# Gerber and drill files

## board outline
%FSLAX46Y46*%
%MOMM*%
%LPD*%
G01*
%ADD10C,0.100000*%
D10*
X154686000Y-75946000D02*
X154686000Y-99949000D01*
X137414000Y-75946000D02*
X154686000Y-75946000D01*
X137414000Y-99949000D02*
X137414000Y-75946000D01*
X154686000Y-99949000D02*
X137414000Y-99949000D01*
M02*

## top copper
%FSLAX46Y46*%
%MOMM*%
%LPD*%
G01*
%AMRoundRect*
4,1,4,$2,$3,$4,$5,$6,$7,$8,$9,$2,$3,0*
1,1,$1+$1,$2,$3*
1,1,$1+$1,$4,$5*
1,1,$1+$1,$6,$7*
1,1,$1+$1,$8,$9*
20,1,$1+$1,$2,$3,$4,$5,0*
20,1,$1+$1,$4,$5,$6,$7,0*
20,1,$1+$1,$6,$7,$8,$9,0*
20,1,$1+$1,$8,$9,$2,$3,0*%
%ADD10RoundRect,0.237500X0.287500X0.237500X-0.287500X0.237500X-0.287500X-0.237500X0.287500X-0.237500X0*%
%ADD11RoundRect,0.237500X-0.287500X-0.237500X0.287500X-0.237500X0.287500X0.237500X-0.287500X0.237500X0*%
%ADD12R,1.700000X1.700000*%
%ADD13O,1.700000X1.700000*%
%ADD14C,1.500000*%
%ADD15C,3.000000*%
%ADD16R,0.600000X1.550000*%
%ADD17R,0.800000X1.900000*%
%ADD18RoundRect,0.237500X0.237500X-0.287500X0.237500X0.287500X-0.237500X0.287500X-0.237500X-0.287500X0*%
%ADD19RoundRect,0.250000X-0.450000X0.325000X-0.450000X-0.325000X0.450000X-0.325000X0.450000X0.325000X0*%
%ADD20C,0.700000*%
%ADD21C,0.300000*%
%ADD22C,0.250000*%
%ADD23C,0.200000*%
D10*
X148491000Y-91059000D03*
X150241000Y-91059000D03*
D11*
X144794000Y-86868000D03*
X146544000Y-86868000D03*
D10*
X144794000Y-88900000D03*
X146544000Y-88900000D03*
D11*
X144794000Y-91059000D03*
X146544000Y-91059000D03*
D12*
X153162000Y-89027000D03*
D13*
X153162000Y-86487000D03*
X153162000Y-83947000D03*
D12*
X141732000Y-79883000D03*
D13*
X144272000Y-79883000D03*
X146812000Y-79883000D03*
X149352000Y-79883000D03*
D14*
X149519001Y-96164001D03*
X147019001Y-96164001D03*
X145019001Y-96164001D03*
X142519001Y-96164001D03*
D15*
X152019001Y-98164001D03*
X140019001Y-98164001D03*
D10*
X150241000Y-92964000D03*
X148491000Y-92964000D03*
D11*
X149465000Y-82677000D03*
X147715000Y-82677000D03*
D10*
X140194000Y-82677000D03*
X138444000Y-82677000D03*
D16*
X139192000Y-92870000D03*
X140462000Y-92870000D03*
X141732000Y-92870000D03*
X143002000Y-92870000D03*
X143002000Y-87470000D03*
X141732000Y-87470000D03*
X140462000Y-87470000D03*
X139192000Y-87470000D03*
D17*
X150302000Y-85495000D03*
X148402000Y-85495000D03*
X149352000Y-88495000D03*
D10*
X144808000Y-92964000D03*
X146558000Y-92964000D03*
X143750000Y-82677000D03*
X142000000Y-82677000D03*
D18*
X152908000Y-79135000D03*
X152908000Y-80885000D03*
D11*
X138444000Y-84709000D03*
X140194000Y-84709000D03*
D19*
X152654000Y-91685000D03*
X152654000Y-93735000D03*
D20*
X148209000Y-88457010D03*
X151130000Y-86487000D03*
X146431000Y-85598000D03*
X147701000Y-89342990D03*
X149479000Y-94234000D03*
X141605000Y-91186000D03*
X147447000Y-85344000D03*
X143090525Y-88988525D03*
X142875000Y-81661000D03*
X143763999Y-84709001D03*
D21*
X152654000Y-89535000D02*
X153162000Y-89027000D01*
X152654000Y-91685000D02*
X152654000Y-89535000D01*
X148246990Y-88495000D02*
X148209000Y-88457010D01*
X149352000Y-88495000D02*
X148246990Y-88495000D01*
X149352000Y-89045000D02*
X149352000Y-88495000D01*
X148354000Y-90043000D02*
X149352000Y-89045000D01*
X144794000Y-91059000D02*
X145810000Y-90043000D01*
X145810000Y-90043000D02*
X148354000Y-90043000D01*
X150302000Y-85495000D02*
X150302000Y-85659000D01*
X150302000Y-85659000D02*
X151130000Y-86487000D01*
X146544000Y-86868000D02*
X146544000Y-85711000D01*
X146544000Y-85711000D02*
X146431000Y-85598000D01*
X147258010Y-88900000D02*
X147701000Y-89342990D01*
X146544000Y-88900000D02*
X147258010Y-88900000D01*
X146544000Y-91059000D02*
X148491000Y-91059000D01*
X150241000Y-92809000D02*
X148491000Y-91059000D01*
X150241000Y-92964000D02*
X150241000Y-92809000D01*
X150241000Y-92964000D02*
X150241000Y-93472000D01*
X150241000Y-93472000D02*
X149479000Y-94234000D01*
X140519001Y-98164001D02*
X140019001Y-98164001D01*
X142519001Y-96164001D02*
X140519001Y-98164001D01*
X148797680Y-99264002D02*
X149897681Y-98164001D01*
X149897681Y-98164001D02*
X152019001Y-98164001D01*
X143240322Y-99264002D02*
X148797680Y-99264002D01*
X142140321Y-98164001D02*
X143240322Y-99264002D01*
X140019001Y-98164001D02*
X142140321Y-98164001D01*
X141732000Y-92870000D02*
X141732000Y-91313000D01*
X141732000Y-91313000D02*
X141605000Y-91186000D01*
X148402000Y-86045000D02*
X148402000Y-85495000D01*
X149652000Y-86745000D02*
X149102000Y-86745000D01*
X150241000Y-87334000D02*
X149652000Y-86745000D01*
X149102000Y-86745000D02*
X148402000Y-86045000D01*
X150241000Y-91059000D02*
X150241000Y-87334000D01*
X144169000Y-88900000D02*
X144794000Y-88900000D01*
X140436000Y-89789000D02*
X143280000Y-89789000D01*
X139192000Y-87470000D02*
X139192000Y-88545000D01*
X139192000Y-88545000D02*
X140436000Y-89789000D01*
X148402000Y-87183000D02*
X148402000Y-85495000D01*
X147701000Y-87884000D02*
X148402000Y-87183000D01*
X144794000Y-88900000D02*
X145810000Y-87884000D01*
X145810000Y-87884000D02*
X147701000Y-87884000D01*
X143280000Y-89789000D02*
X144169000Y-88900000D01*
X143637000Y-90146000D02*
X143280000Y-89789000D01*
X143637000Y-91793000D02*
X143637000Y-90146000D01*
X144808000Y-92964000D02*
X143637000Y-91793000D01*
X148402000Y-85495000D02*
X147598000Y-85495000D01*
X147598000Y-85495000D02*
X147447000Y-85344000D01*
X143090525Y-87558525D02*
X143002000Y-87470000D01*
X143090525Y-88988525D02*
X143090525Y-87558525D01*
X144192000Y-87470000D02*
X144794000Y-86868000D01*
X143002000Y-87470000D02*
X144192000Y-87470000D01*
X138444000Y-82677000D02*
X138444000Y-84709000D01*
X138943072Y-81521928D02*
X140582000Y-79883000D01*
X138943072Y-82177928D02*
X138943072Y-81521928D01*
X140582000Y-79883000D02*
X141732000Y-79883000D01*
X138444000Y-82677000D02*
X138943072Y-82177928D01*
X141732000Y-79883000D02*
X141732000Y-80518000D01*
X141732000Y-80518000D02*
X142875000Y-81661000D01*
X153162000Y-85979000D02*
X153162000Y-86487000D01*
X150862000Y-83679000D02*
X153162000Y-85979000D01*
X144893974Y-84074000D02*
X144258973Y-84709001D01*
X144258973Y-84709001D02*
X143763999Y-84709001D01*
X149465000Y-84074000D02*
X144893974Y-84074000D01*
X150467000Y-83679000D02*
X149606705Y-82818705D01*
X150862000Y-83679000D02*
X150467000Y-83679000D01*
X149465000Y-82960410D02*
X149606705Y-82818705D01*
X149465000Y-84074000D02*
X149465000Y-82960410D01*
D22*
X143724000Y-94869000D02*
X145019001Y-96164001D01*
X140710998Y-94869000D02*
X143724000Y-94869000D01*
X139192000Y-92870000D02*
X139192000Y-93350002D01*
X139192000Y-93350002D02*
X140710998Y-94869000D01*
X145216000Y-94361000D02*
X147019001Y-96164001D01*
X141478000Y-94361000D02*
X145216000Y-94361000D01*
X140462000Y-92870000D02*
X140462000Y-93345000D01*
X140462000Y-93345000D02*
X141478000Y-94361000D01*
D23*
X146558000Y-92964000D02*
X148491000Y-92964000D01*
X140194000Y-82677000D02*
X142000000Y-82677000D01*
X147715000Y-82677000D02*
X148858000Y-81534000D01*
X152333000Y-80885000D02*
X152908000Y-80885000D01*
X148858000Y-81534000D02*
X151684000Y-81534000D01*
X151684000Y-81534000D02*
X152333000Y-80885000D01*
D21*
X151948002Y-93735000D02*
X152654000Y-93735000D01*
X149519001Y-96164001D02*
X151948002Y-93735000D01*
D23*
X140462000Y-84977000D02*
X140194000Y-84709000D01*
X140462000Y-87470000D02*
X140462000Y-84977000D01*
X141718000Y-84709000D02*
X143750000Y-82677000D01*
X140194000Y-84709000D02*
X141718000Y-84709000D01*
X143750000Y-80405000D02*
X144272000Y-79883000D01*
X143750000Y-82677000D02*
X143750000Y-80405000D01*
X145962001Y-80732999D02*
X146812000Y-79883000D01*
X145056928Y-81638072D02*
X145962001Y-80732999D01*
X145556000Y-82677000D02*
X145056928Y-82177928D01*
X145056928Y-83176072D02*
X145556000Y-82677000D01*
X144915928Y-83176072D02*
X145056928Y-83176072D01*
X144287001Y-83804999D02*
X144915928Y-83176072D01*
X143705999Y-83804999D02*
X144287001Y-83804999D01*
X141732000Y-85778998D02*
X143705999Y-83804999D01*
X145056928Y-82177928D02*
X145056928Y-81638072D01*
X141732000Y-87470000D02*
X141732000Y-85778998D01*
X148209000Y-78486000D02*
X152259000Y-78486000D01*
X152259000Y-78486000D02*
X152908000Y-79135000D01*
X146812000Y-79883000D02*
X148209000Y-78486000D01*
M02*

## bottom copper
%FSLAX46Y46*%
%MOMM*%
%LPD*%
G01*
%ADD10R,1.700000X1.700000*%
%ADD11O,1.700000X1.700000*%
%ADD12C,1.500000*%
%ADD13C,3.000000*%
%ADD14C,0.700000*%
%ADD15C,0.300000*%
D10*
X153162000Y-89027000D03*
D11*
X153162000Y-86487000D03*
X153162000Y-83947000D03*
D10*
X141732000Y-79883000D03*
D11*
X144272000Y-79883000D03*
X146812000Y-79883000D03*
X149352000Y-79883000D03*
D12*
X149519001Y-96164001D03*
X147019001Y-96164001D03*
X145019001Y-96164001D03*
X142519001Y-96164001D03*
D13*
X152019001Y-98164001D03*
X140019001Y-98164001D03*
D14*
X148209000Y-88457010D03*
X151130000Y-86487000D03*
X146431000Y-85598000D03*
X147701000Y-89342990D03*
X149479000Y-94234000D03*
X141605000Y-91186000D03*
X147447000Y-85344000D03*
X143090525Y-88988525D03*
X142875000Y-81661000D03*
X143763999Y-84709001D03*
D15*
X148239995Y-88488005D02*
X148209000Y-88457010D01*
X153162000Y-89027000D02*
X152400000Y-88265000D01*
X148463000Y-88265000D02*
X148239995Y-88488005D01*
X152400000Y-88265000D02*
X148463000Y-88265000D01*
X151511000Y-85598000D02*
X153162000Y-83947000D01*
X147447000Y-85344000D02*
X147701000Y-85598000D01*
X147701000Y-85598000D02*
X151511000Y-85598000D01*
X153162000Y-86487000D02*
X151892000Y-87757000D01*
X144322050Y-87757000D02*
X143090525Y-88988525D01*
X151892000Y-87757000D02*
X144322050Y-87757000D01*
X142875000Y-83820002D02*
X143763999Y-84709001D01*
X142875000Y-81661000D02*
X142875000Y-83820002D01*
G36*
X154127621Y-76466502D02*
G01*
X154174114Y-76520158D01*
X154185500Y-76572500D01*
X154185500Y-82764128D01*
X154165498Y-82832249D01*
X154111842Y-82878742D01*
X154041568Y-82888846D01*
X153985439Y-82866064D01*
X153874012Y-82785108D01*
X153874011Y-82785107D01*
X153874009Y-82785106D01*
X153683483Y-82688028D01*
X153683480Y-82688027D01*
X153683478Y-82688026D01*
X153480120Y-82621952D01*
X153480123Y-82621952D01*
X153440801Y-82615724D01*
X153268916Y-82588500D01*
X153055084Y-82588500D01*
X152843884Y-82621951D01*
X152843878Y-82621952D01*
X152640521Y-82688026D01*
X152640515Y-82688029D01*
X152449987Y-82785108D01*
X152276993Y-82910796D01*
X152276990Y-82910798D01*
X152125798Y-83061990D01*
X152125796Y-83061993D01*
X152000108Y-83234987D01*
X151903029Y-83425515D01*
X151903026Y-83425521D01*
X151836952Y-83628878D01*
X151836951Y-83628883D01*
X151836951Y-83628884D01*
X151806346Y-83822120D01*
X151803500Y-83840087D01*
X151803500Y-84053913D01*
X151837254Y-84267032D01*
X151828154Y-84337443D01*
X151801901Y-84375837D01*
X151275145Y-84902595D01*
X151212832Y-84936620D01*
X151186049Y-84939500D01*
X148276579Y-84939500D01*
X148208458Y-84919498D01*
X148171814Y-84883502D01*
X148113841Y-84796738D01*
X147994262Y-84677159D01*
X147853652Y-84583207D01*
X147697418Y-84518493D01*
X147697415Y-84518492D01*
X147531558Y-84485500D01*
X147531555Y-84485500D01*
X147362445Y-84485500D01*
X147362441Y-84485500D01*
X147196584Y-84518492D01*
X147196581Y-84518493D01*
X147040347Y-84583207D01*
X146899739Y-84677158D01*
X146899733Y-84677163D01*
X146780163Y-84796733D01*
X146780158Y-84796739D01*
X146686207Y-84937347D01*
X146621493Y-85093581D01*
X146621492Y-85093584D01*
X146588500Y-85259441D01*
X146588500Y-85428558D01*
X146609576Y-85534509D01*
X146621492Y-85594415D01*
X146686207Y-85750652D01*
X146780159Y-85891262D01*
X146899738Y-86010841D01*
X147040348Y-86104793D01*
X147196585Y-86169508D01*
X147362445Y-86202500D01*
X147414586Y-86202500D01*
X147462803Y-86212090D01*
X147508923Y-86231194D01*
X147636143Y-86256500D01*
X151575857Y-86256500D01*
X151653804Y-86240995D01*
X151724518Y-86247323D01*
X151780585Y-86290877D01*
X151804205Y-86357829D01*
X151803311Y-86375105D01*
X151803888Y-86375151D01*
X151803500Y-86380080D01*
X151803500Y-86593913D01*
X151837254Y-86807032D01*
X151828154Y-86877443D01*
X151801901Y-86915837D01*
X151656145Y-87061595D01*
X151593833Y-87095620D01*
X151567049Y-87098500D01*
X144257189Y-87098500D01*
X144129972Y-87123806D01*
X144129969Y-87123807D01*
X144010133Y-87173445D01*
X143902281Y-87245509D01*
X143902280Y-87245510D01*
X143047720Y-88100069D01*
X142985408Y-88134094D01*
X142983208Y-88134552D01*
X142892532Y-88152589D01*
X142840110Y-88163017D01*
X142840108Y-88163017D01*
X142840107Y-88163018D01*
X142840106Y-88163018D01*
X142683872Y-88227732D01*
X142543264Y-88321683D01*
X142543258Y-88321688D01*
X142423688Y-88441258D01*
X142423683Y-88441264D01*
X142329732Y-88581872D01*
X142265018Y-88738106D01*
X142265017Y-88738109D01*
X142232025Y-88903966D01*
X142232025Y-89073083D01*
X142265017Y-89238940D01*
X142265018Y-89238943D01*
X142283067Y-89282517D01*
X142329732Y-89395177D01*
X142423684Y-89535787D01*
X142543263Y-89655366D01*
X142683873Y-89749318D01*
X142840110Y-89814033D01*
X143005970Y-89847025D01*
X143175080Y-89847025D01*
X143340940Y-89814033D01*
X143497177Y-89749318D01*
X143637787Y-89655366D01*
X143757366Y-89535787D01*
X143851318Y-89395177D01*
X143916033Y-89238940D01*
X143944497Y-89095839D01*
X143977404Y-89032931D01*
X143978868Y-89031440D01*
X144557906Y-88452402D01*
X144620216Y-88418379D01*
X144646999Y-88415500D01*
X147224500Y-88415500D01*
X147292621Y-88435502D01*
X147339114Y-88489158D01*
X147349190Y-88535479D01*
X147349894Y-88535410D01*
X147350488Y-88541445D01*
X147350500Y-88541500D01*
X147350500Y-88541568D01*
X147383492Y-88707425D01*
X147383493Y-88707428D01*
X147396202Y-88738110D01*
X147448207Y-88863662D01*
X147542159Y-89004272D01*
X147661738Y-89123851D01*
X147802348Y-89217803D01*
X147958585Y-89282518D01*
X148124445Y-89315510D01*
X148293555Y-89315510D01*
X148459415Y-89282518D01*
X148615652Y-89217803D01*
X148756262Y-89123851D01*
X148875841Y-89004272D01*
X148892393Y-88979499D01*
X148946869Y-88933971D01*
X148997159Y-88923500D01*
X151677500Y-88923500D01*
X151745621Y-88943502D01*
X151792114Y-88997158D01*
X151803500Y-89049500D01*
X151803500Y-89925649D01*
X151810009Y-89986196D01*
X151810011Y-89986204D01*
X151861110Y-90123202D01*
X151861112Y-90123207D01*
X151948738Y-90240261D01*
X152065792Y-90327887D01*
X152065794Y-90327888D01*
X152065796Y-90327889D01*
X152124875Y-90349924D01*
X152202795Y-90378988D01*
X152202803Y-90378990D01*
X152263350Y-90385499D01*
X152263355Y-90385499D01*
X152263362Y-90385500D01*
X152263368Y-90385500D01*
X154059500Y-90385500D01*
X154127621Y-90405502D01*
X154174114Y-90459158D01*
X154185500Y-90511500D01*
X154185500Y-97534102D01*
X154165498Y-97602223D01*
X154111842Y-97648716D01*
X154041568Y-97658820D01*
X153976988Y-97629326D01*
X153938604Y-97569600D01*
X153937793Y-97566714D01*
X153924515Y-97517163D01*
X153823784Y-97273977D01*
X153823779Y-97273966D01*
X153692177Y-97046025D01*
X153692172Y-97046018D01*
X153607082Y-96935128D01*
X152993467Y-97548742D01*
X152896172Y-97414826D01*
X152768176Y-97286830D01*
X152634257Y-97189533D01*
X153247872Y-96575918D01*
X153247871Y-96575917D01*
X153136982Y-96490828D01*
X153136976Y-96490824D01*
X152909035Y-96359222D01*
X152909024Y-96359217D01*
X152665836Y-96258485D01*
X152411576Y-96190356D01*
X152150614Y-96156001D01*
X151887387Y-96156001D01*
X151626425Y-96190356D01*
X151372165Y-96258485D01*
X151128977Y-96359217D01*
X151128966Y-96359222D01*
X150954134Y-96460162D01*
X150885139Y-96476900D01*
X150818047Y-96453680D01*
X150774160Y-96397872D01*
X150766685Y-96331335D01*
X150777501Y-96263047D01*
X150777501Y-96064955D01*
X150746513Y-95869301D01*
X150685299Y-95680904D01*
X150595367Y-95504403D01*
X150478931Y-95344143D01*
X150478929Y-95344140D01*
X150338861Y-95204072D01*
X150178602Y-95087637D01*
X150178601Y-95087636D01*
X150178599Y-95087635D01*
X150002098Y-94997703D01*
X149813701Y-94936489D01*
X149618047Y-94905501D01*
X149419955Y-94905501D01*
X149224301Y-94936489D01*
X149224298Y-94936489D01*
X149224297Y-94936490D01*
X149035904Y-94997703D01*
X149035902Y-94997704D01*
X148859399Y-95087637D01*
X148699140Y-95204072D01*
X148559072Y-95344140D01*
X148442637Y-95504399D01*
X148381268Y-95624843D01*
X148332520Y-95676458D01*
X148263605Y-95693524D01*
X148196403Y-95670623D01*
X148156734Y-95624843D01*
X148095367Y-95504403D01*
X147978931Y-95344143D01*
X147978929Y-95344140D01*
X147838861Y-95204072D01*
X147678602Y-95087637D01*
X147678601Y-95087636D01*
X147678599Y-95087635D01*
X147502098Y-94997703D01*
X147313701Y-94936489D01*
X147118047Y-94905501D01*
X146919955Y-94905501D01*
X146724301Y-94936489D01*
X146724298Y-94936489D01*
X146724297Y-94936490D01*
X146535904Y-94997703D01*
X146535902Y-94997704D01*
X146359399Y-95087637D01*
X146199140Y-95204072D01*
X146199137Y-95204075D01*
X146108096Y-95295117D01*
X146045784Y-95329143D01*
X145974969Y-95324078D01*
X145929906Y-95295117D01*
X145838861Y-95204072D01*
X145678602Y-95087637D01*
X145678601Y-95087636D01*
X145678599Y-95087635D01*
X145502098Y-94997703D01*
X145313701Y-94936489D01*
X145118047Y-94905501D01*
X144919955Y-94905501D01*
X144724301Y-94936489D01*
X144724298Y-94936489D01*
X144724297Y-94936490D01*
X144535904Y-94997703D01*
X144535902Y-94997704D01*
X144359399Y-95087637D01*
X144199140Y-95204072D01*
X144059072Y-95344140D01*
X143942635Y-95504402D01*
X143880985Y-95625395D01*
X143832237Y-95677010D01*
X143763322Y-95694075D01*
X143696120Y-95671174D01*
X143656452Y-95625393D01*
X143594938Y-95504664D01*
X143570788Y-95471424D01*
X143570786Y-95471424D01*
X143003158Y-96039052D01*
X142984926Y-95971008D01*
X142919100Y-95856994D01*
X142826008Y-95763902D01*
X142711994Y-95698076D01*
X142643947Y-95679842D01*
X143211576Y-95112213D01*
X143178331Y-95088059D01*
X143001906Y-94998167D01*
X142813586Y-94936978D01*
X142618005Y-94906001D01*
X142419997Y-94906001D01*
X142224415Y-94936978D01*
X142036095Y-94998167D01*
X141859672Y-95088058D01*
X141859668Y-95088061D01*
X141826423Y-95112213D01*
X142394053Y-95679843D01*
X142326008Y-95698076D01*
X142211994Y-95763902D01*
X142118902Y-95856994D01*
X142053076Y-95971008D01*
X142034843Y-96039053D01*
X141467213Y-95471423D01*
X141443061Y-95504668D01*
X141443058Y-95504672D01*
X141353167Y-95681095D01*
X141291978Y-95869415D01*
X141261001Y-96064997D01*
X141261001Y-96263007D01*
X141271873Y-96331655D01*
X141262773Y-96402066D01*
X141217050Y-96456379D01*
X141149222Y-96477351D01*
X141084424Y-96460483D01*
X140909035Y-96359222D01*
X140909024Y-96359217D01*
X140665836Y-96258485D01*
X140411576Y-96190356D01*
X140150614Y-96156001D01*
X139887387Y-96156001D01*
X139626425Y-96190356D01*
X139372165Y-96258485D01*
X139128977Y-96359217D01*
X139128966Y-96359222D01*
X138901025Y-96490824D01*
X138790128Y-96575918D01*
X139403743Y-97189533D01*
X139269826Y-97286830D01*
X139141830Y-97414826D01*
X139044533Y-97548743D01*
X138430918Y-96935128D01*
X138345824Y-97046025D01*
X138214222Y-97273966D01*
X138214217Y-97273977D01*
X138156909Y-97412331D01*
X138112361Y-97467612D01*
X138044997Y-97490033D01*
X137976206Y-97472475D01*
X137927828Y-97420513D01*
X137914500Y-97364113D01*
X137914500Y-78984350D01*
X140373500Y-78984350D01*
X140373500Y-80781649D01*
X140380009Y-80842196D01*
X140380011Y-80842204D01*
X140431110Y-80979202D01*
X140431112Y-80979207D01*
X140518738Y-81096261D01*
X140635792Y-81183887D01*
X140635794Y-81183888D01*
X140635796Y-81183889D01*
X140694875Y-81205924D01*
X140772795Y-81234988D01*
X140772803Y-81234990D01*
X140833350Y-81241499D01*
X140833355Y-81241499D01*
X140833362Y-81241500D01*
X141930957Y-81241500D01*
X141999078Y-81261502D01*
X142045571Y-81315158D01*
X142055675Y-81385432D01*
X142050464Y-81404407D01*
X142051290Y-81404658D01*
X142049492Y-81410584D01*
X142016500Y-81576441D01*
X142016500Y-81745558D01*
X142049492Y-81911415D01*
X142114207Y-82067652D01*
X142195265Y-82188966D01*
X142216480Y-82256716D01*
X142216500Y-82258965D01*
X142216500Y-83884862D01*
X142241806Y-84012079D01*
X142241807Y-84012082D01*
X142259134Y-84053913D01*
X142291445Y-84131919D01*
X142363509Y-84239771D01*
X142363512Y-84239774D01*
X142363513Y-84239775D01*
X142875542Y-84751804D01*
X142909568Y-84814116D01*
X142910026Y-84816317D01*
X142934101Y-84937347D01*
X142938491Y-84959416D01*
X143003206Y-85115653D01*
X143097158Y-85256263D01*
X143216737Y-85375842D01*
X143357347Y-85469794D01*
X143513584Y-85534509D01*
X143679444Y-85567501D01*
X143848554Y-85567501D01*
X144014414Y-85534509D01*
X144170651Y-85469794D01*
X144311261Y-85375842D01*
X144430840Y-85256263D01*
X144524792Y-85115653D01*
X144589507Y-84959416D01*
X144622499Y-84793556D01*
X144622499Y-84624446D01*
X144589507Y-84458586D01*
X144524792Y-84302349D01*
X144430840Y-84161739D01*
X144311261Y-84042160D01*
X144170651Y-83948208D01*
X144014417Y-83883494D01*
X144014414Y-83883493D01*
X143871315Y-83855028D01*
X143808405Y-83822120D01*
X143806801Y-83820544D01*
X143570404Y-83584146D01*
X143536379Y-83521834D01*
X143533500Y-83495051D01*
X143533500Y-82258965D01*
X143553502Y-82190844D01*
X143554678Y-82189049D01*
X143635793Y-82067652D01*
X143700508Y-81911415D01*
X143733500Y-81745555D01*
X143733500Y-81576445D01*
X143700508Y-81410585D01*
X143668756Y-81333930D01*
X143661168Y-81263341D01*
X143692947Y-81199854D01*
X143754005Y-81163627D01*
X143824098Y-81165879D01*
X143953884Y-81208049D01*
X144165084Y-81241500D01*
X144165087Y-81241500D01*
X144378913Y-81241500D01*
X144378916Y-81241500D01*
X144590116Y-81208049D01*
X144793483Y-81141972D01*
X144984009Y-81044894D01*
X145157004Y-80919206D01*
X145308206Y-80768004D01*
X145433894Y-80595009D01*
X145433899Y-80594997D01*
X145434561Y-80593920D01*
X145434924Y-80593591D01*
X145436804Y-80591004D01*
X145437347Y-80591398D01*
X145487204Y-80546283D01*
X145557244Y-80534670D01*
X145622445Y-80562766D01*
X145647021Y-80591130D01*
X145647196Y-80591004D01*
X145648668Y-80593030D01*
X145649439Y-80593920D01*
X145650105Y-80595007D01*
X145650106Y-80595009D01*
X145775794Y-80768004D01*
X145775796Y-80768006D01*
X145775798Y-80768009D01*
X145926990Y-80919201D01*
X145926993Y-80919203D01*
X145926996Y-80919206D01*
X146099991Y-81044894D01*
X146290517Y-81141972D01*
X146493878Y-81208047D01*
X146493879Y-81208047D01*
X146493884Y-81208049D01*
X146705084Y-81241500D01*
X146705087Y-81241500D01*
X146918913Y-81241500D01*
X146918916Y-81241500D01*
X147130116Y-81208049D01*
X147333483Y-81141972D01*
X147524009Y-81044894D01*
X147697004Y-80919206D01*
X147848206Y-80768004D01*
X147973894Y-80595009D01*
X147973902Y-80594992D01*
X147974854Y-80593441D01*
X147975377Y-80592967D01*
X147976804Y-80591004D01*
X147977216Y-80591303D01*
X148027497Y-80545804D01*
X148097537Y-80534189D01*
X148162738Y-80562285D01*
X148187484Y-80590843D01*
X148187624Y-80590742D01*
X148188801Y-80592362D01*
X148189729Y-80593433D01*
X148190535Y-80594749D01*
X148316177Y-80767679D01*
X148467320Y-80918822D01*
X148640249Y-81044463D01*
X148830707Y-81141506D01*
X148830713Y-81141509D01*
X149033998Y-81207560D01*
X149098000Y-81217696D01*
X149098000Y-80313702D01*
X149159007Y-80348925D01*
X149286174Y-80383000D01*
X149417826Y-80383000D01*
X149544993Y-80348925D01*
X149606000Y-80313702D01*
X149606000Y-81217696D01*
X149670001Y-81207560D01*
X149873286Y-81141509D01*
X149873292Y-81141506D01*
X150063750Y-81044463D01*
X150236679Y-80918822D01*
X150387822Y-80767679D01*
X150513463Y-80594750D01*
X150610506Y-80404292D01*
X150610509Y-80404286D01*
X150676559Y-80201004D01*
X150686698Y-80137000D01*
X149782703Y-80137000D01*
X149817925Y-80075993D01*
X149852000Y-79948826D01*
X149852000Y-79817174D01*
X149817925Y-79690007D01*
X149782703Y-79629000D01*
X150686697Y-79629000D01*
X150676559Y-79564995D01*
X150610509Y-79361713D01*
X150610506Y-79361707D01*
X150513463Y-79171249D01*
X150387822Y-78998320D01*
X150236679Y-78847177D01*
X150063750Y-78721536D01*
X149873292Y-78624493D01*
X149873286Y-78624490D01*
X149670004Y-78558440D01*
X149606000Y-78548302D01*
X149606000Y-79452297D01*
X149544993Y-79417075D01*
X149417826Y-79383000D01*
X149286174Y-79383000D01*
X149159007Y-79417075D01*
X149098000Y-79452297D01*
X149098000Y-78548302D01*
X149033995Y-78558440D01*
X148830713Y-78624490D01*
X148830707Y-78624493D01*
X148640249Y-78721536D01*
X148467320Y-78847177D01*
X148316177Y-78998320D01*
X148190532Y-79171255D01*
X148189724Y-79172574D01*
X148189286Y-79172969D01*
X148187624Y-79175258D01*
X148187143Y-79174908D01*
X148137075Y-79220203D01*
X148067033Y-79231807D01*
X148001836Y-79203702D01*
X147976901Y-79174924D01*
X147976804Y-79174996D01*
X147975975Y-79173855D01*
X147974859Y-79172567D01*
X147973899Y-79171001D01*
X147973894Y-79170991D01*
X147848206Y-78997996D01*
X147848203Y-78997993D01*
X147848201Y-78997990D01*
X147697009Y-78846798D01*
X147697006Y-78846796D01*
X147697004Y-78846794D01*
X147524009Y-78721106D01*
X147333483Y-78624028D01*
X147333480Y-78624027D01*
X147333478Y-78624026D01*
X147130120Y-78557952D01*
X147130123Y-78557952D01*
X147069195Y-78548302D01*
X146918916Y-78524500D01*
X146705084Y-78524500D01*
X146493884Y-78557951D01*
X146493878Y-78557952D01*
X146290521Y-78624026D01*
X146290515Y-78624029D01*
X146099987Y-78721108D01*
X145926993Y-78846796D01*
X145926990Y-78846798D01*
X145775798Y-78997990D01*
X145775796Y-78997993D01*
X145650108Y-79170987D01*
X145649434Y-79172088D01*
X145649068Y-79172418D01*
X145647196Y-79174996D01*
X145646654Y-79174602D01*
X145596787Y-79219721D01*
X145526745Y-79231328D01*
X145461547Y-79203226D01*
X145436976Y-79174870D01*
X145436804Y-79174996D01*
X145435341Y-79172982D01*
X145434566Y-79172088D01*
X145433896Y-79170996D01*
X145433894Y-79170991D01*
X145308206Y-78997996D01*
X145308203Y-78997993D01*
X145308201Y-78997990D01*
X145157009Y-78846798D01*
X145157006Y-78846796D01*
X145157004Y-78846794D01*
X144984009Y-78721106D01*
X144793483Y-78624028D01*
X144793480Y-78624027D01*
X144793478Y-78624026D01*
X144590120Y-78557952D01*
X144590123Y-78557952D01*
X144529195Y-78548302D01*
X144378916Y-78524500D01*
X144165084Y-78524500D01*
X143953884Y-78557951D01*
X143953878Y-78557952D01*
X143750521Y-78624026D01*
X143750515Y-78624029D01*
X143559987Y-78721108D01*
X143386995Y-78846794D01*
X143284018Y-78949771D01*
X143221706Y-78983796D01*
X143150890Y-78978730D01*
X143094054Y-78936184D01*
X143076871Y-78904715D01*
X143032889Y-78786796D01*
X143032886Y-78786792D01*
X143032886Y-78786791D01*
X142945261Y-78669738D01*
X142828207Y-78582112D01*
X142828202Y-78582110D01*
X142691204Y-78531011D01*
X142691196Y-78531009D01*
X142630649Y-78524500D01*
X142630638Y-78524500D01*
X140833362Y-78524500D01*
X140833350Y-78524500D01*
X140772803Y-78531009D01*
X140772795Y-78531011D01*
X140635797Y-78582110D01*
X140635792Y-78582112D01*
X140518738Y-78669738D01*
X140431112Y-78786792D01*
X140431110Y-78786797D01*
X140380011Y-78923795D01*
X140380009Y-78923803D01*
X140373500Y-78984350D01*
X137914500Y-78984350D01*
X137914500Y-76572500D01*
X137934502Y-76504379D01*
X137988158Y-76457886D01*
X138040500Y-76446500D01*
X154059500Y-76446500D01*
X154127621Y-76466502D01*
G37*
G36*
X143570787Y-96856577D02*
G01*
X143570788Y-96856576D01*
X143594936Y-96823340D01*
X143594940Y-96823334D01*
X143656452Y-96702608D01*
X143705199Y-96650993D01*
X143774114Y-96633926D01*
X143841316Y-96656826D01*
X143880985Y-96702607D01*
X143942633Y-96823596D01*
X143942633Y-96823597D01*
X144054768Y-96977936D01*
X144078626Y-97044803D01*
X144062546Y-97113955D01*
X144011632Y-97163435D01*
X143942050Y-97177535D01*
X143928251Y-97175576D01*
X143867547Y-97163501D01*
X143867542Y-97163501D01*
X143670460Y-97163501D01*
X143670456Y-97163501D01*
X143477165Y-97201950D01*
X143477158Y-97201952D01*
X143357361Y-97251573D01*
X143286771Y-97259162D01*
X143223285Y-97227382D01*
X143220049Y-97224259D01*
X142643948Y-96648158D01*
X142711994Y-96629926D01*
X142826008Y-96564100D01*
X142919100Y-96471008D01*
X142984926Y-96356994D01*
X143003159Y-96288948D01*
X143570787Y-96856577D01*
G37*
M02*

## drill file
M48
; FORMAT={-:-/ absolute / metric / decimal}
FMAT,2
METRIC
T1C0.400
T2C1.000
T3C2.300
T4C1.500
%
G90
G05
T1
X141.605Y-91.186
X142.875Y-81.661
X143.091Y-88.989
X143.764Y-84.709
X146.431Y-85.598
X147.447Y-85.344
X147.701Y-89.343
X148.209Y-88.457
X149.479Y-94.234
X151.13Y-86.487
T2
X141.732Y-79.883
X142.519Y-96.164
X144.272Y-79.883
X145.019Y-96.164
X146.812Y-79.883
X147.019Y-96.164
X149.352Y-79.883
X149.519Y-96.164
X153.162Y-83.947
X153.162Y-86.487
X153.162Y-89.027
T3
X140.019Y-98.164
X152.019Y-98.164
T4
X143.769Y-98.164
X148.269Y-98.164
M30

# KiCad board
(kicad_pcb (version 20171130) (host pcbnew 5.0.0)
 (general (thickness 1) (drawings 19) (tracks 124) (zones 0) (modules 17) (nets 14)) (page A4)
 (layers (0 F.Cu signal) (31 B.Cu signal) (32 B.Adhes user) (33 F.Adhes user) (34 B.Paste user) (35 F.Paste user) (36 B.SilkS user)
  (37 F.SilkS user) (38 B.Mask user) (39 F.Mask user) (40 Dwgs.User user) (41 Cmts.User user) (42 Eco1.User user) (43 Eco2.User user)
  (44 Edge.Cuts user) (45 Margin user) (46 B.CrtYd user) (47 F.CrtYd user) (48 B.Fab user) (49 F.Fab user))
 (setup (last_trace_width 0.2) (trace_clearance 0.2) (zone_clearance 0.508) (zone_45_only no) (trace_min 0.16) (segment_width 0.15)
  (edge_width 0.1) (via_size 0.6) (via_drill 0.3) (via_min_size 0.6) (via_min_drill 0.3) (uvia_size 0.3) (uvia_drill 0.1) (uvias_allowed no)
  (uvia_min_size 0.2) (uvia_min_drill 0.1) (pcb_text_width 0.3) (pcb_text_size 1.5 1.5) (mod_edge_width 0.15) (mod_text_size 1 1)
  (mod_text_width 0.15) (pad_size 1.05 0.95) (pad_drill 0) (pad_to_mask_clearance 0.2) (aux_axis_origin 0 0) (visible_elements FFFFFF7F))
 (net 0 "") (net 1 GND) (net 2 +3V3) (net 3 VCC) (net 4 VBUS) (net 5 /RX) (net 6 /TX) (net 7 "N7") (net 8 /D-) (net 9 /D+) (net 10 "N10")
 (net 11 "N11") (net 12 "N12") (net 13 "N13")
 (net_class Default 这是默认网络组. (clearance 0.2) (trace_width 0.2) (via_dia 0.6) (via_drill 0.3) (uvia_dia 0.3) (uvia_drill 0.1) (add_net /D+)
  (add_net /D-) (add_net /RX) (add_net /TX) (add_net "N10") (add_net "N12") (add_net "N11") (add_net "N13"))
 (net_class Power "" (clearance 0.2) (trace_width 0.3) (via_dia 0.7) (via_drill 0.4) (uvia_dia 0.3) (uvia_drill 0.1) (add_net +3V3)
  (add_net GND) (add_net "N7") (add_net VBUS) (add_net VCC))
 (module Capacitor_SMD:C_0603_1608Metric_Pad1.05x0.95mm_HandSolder (layer F.Cu) (at 149.366 91.059 180)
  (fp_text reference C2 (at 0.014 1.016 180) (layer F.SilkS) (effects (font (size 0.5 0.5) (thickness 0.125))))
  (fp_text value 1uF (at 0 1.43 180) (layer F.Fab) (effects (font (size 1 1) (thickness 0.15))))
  (pad 2 smd roundrect (at 0.875 0 180) (size 1.05 0.95) (layers F.Cu F.Paste F.Mask) (roundrect_rratio 0.25) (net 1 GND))
  (pad 1 smd roundrect (at -0.875 0 180) (size 1.05 0.95) (layers F.Cu F.Paste F.Mask) (roundrect_rratio 0.25) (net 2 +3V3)))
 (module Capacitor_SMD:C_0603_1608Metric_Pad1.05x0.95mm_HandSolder (layer F.Cu) (at 145.669 86.868)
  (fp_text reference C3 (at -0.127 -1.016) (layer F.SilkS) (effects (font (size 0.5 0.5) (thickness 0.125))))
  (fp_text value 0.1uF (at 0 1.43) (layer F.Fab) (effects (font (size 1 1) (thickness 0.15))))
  (pad 1 smd roundrect (at -0.875 0) (size 1.05 0.95) (layers F.Cu F.Paste F.Mask) (roundrect_rratio 0.25) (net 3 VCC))
  (pad 2 smd roundrect (at 0.875 0) (size 1.05 0.95) (layers F.Cu F.Paste F.Mask) (roundrect_rratio 0.25) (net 1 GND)))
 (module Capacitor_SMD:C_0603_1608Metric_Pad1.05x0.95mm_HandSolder (layer F.Cu) (at 145.669 88.9 180)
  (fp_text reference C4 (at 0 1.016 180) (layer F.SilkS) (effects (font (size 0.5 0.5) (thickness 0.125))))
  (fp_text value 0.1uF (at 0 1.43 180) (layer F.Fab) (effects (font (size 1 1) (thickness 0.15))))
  (pad 2 smd roundrect (at 0.875 0 180) (size 1.05 0.95) (layers F.Cu F.Paste F.Mask) (roundrect_rratio 0.25) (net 2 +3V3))
  (pad 1 smd roundrect (at -0.875 0 180) (size 1.05 0.95) (layers F.Cu F.Paste F.Mask) (roundrect_rratio 0.25) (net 1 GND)))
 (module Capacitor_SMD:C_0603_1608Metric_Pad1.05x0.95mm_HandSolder (layer F.Cu) (at 145.669 91.059)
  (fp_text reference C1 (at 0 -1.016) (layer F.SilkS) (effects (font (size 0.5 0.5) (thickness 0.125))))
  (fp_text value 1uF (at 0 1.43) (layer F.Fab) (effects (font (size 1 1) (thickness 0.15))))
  (pad 1 smd roundrect (at -0.875 0) (size 1.05 0.95) (layers F.Cu F.Paste F.Mask) (roundrect_rratio 0.25) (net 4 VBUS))
  (pad 2 smd roundrect (at 0.875 0) (size 1.05 0.95) (layers F.Cu F.Paste F.Mask) (roundrect_rratio 0.25) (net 1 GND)))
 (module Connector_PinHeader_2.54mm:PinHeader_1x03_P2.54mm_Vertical (layer F.Cu) (at 153.162 89.027 180)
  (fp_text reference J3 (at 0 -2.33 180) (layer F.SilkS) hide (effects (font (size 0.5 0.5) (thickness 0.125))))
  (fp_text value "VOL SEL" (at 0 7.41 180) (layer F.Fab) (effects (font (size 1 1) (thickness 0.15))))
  (pad 1 thru_hole rect (at 0 0 180) (size 1.7 1.7) (drill 1) (layers *.Cu *.Mask) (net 4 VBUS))
  (pad 2 thru_hole oval (at 0 2.54 180) (size 1.7 1.7) (drill 1) (layers *.Cu *.Mask) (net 3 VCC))
  (pad 3 thru_hole oval (at 0 5.08 180) (size 1.7 1.7) (drill 1) (layers *.Cu *.Mask) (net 2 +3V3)))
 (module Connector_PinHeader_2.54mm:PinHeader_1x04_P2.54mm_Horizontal (layer F.Cu) (at 141.732 79.883 90)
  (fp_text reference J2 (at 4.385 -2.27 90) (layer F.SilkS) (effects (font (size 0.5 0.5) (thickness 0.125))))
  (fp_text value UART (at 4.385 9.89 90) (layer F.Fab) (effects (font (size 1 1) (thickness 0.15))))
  (pad 1 thru_hole rect (at 0 0 90) (size 1.7 1.7) (drill 1) (layers *.Cu *.Mask) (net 3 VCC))
  (pad 2 thru_hole oval (at 0 2.54 90) (size 1.7 1.7) (drill 1) (layers *.Cu *.Mask) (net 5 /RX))
  (pad 3 thru_hole oval (at 0 5.08 90) (size 1.7 1.7) (drill 1) (layers *.Cu *.Mask) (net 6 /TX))
  (pad 4 thru_hole oval (at 0 7.62 90) (size 1.7 1.7) (drill 1) (layers *.Cu *.Mask) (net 1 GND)))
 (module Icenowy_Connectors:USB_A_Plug (layer F.Cu) (at 142.519001 96.164001)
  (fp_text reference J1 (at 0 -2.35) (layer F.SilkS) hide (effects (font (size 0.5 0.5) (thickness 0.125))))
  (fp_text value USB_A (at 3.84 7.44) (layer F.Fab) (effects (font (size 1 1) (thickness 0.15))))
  (pad "" np_thru_hole circle (at 5.75 2 270) (size 1.5 1.5) (drill 1.5) (layers *.Cu *.Mask))
  (pad 1 thru_hole circle (at 7 0 270) (size 1.5 1.5) (drill 1) (layers *.Cu *.Mask) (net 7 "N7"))
  (pad 2 thru_hole circle (at 4.5 0 270) (size 1.5 1.5) (drill 1) (layers *.Cu *.Mask) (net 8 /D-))
  (pad 3 thru_hole circle (at 2.5 0 270) (size 1.5 1.5) (drill 1) (layers *.Cu *.Mask) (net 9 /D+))
  (pad 4 thru_hole circle (at 0 0 270) (size 1.5 1.5) (drill 1) (layers *.Cu *.Mask) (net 1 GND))
  (pad 5 thru_hole circle (at 9.5 2 270) (size 3 3) (drill 2.3) (layers *.Cu *.Mask) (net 1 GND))
  (pad 5 thru_hole circle (at -2.5 2 270) (size 3 3) (drill 2.3) (layers *.Cu *.Mask) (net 1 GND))
  (pad "" np_thru_hole circle (at 1.25 2 270) (size 1.5 1.5) (drill 1.5) (layers *.Cu *.Mask)))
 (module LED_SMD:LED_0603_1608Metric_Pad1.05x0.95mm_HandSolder (layer F.Cu) (at 149.366 92.964 180)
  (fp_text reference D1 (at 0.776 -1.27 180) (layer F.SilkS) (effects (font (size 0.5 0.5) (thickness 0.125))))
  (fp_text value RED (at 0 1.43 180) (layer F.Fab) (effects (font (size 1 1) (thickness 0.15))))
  (pad 1 smd roundrect (at -0.875 0 180) (size 1.05 0.95) (layers F.Cu F.Paste F.Mask) (roundrect_rratio 0.25) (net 1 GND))
  (pad 2 smd roundrect (at 0.875 0 180) (size 1.05 0.95) (layers F.Cu F.Paste F.Mask) (roundrect_rratio 0.25) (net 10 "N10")))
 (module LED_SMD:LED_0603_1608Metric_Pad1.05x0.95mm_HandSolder (layer F.Cu) (at 148.59 82.677)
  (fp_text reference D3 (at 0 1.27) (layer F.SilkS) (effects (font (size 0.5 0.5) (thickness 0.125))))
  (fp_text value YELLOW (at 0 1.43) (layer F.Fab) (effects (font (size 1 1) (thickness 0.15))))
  (pad 2 smd roundrect (at 0.875 0) (size 1.05 0.95) (layers F.Cu F.Paste F.Mask) (roundrect_rratio 0.25) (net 3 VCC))
  (pad 1 smd roundrect (at -0.875 0) (size 1.05 0.95) (layers F.Cu F.Paste F.Mask) (roundrect_rratio 0.25) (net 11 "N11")))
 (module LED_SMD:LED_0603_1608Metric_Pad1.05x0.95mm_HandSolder (layer F.Cu) (at 139.319 82.677 180)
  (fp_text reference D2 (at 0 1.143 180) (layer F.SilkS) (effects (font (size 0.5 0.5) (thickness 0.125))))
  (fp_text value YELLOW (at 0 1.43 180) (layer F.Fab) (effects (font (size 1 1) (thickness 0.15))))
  (pad 1 smd roundrect (at -0.875 0 180) (size 1.05 0.95) (layers F.Cu F.Paste F.Mask) (roundrect_rratio 0.25) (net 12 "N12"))
  (pad 2 smd roundrect (at 0.875 0 180) (size 1.05 0.95) (layers F.Cu F.Paste F.Mask) (roundrect_rratio 0.25) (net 3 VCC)))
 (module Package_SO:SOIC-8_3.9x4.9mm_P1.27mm (layer F.Cu) (at 141.097 90.17 90)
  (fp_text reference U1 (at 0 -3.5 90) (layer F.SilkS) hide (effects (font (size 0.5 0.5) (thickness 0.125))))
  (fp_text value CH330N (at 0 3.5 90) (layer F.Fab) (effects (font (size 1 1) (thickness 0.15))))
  (pad 1 smd rect (at -2.7 -1.905 90) (size 1.55 0.6) (layers F.Cu F.Paste F.Mask) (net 9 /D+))
  (pad 2 smd rect (at -2.7 -0.635 90) (size 1.55 0.6) (layers F.Cu F.Paste F.Mask) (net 8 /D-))
  (pad 3 smd rect (at -2.7 0.635 90) (size 1.55 0.6) (layers F.Cu F.Paste F.Mask) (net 1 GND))
  (pad 4 smd rect (at -2.7 1.905 90) (size 1.55 0.6) (layers F.Cu F.Paste F.Mask) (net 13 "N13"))
  (pad 5 smd rect (at 2.7 1.905 90) (size 1.55 0.6) (layers F.Cu F.Paste F.Mask) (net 3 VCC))
  (pad 6 smd rect (at 2.7 0.635 90) (size 1.55 0.6) (layers F.Cu F.Paste F.Mask) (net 6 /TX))
  (pad 7 smd rect (at 2.7 -0.635 90) (size 1.55 0.6) (layers F.Cu F.Paste F.Mask) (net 5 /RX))
  (pad 8 smd rect (at 2.7 -1.905 90) (size 1.55 0.6) (layers F.Cu F.Paste F.Mask) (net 2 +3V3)))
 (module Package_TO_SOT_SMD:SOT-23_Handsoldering (layer F.Cu) (at 149.352 86.995 270)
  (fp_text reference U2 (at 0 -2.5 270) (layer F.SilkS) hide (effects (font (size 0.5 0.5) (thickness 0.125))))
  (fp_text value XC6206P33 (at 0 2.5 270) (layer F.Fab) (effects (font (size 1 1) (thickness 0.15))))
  (pad 1 smd rect (at -1.5 -0.95 270) (size 1.9 0.8) (layers F.Cu F.Paste F.Mask) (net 1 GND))
  (pad 2 smd rect (at -1.5 0.95 270) (size 1.9 0.8) (layers F.Cu F.Paste F.Mask) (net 2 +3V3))
  (pad 3 smd rect (at 1.5 0 270) (size 1.9 0.8) (layers F.Cu F.Paste F.Mask) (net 4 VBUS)))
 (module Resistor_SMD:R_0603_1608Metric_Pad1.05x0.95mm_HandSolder (layer F.Cu) (at 145.683 92.964 180)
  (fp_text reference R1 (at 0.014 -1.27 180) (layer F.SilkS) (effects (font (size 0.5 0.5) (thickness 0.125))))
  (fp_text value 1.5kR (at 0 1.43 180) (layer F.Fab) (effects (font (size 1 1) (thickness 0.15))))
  (pad 2 smd roundrect (at 0.875 0 180) (size 1.05 0.95) (layers F.Cu F.Paste F.Mask) (roundrect_rratio 0.25) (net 2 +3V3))
  (pad 1 smd roundrect (at -0.875 0 180) (size 1.05 0.95) (layers F.Cu F.Paste F.Mask) (roundrect_rratio 0.25) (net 10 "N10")))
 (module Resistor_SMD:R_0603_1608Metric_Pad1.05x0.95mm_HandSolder (layer F.Cu) (at 142.875 82.677 180)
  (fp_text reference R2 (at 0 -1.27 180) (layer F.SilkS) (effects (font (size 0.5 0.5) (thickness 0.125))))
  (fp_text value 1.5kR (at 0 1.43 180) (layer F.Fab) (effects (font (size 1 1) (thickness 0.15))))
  (pad 1 smd roundrect (at -0.875 0 180) (size 1.05 0.95) (layers F.Cu F.Paste F.Mask) (roundrect_rratio 0.25) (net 5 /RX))
  (pad 2 smd roundrect (at 0.875 0 180) (size 1.05 0.95) (layers F.Cu F.Paste F.Mask) (roundrect_rratio 0.25) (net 12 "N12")))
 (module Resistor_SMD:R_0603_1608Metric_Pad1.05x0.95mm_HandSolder (layer F.Cu) (at 152.908 80.01 90)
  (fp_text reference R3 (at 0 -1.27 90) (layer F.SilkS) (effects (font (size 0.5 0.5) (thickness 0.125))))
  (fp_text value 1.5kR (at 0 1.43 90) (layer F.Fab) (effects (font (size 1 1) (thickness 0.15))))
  (pad 2 smd roundrect (at 0.875 0 90) (size 1.05 0.95) (layers F.Cu F.Paste F.Mask) (roundrect_rratio 0.25) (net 6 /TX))
  (pad 1 smd roundrect (at -0.875 0 90) (size 1.05 0.95) (layers F.Cu F.Paste F.Mask) (roundrect_rratio 0.25) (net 11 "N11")))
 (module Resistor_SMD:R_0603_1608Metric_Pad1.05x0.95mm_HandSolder (layer F.Cu) (at 139.319 84.709)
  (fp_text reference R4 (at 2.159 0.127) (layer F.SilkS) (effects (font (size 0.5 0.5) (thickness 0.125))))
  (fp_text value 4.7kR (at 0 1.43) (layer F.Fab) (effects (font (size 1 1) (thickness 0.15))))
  (pad 1 smd roundrect (at -0.875 0) (size 1.05 0.95) (layers F.Cu F.Paste F.Mask) (roundrect_rratio 0.25) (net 3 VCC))
  (pad 2 smd roundrect (at 0.875 0) (size 1.05 0.95) (layers F.Cu F.Paste F.Mask) (roundrect_rratio 0.25) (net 5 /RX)))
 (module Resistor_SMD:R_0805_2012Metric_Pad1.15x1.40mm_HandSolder (layer F.Cu) (at 152.654 92.71 270)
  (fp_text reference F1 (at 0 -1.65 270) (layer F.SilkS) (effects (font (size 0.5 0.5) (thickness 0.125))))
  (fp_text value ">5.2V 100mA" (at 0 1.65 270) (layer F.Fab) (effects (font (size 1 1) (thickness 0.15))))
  (pad 1 smd roundrect (at -1.025 0 270) (size 1.15 1.4) (layers F.Cu F.Paste F.Mask) (roundrect_rratio 0.217391) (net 4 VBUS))
  (pad 2 smd roundrect (at 1.025 0 270) (size 1.15 1.4) (layers F.Cu F.Paste F.Mask) (roundrect_rratio 0.217391) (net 7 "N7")))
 (gr_line (start 154.686 75.946) (end 154.686 99.949) (layer Edge.Cuts) (width 0.1))
 (gr_line (start 137.414 75.946) (end 154.686 75.946) (layer Edge.Cuts) (width 0.1))
 (gr_line (start 137.414 99.949) (end 137.414 75.946) (layer Edge.Cuts) (width 0.1))
 (gr_line (start 154.686 99.949) (end 137.414 99.949) (layer Edge.Cuts) (width 0.1))
 (segment (start 152.654 89.535) (end 153.162 89.027) (width 0.3) (layer F.Cu) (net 4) (status 30))
 (segment (start 152.654 91.685) (end 152.654 89.535) (width 0.3) (layer F.Cu) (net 4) (status 30))
 (segment (start 148.24699 88.495) (end 148.209 88.45701) (width 0.3) (layer F.Cu) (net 4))
 (segment (start 149.352 88.495) (end 148.24699 88.495) (width 0.3) (layer F.Cu) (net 4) (status 10))
 (via (at 148.209 88.45701) (size 0.7) (drill 0.4) (layers F.Cu B.Cu) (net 4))
 (segment (start 149.352 89.045) (end 149.352 88.495) (width 0.3) (layer F.Cu) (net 4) (status 30))
 (segment (start 148.354 90.043) (end 149.352 89.045) (width 0.3) (layer F.Cu) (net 4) (status 20))
 (segment (start 144.794 91.059) (end 145.81 90.043) (width 0.3) (layer F.Cu) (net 4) (status 10))
 (segment (start 145.81 90.043) (end 148.354 90.043) (width 0.3) (layer F.Cu) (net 4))
 (segment (start 148.239995 88.488005) (end 148.209 88.45701) (width 0.3) (layer B.Cu) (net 4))
 (segment (start 153.162 89.027) (end 152.4 88.265) (width 0.3) (layer B.Cu) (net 4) (status 30))
 (segment (start 148.463 88.265) (end 148.239995 88.488005) (width 0.3) (layer B.Cu) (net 4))
 (segment (start 152.4 88.265) (end 148.463 88.265) (width 0.3) (layer B.Cu) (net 4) (status 10))
 (via (at 151.13 86.487) (size 0.7) (drill 0.4) (layers F.Cu B.Cu) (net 1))
 (segment (start 150.302 85.495) (end 150.302 85.659) (width 0.3) (layer F.Cu) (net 1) (status 30))
 (segment (start 150.302 85.659) (end 151.13 86.487) (width 0.3) (layer F.Cu) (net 1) (status 10))
 (via (at 146.431 85.598) (size 0.7) (drill 0.4) (layers F.Cu B.Cu) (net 1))
 (segment (start 146.544 86.868) (end 146.544 85.711) (width 0.3) (layer F.Cu) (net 1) (status 10))
 (segment (start 146.544 85.711) (end 146.431 85.598) (width 0.3) (layer F.Cu) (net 1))
 (segment (start 147.25801 88.9) (end 147.701 89.34299) (width 0.3) (layer F.Cu) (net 1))
 (segment (start 146.544 88.9) (end 147.25801 88.9) (width 0.3) (layer F.Cu) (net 1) (status 10))
 (via (at 147.701 89.34299) (size 0.7) (drill 0.4) (layers F.Cu B.Cu) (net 1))
 (segment (start 146.544 91.059) (end 148.491 91.059) (width 0.3) (layer F.Cu) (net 1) (status 30))
 (segment (start 150.241 92.809) (end 148.491 91.059) (width 0.3) (layer F.Cu) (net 1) (status 30))
 (segment (start 150.241 92.964) (end 150.241 92.809) (width 0.3) (layer F.Cu) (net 1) (status 30))
 (segment (start 150.241 92.964) (end 150.241 93.472) (width 0.3) (layer F.Cu) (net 1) (status 10))
 (via (at 149.479 94.234) (size 0.7) (drill 0.4) (layers F.Cu B.Cu) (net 1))
 (segment (start 150.241 93.472) (end 149.479 94.234) (width 0.3) (layer F.Cu) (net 1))
 (segment (start 140.519001 98.164001) (end 140.019001 98.164001) (width 0.3) (layer F.Cu) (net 1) (status 30))
 (segment (start 142.519001 96.164001) (end 140.519001 98.164001) (width 0.3) (layer F.Cu) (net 1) (status 30))
 (segment (start 148.79768 99.264002) (end 149.897681 98.164001) (width 0.3) (layer F.Cu) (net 1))
 (segment (start 149.897681 98.164001) (end 152.019001 98.164001) (width 0.3) (layer F.Cu) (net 1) (status 20))
 (segment (start 143.240322 99.264002) (end 148.79768 99.264002) (width 0.3) (layer F.Cu) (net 1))
 (segment (start 142.140321 98.164001) (end 143.240322 99.264002) (width 0.3) (layer F.Cu) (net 1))
 (segment (start 140.019001 98.164001) (end 142.140321 98.164001) (width 0.3) (layer F.Cu) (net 1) (status 10))
 (segment (start 141.732 92.87) (end 141.732 91.313) (width 0.3) (layer F.Cu) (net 1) (status 10))
 (via (at 141.605 91.186) (size 0.7) (drill 0.4) (layers F.Cu B.Cu) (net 1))
 (segment (start 141.732 91.313) (end 141.605 91.186) (width 0.3) (layer F.Cu) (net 1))
 (segment (start 148.402 86.045) (end 148.402 85.495) (width 0.3) (layer F.Cu) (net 2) (status 30))
 (segment (start 149.652 86.745) (end 149.102 86.745) (width 0.3) (layer F.Cu) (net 2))
 (segment (start 150.241 87.334) (end 149.652 86.745) (width 0.3) (layer F.Cu) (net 2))
 (segment (start 149.102 86.745) (end 148.402 86.045) (width 0.3) (layer F.Cu) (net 2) (status 20))
 (segment (start 150.241 91.059) (end 150.241 87.334) (width 0.3) (layer F.Cu) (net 2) (status 10))
 (segment (start 144.169 88.9) (end 144.794 88.9) (width 0.3) (layer F.Cu) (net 2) (status 20))
 (segment (start 140.436 89.789) (end 143.28 89.789) (width 0.3) (layer F.Cu) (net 2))
 (segment (start 139.192 87.47) (end 139.192 88.545) (width 0.3) (layer F.Cu) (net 2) (status 10))
 (segment (start 139.192 88.545) (end 140.436 89.789) (width 0.3) (layer F.Cu) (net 2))
 (segment (start 148.402 87.183) (end 148.402 85.495) (width 0.3) (layer F.Cu) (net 2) (status 20))
 (segment (start 147.701 87.884) (end 148.402 87.183) (width 0.3) (layer F.Cu) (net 2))
 (segment (start 144.794 88.9) (end 145.81 87.884) (width 0.3) (layer F.Cu) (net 2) (status 10))
 (segment (start 145.81 87.884) (end 147.701 87.884) (width 0.3) (layer F.Cu) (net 2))
 (segment (start 143.28 89.789) (end 144.169 88.9) (width 0.3) (layer F.Cu) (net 2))
 (segment (start 143.637 90.146) (end 143.28 89.789) (width 0.3) (layer F.Cu) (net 2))
 (segment (start 143.637 91.793) (end 143.637 90.146) (width 0.3) (layer F.Cu) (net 2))
 (segment (start 144.808 92.964) (end 143.637 91.793) (width 0.3) (layer F.Cu) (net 2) (status 10))
 (via (at 147.447 85.344) (size 0.7) (drill 0.4) (layers F.Cu B.Cu) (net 2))
 (segment (start 148.402 85.495) (end 147.598 85.495) (width 0.3) (layer F.Cu) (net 2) (status 10))
 (segment (start 147.598 85.495) (end 147.447 85.344) (width 0.3) (layer F.Cu) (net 2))
 (segment (start 151.511 85.598) (end 153.162 83.947) (width 0.3) (layer B.Cu) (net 2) (status 20))
 (segment (start 147.447 85.344) (end 147.701 85.598) (width 0.3) (layer B.Cu) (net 2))
 (segment (start 147.701 85.598) (end 151.511 85.598) (width 0.3) (layer B.Cu) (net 2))
 (via (at 143.090525 88.988525) (size 0.7) (drill 0.4) (layers F.Cu B.Cu) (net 3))
 (segment (start 143.090525 87.558525) (end 143.002 87.47) (width 0.3) (layer F.Cu) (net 3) (status 30))
 (segment (start 143.090525 88.988525) (end 143.090525 87.558525) (width 0.3) (layer F.Cu) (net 3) (status 20))
 (segment (start 153.162 86.487) (end 151.892 87.757) (width 0.3) (layer B.Cu) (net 3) (status 10))
 (segment (start 144.32205 87.757) (end 143.090525 88.988525) (width 0.3) (layer B.Cu) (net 3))
 (segment (start 151.892 87.757) (end 144.32205 87.757) (width 0.3) (layer B.Cu) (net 3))
 (segment (start 144.192 87.47) (end 144.794 86.868) (width 0.3) (layer F.Cu) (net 3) (status 20))
 (segment (start 143.002 87.47) (end 144.192 87.47) (width 0.3) (layer F.Cu) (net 3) (status 10))
 (segment (start 138.444 82.677) (end 138.444 84.709) (width 0.3) (layer F.Cu) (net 3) (status 30))
 (segment (start 138.943072 81.521928) (end 140.582 79.883) (width 0.3) (layer F.Cu) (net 3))
 (segment (start 138.943072 82.177928) (end 138.943072 81.521928) (width 0.3) (layer F.Cu) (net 3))
 (segment (start 140.582 79.883) (end 141.732 79.883) (width 0.3) (layer F.Cu) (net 3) (status 20))
 (segment (start 138.444 82.677) (end 138.943072 82.177928) (width 0.3) (layer F.Cu) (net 3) (status 10))
 (via (at 142.875 81.661) (size 0.7) (drill 0.4) (layers F.Cu B.Cu) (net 3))
 (segment (start 141.732 79.883) (end 141.732 80.518) (width 0.3) (layer F.Cu) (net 3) (status 30))
 (segment (start 141.732 80.518) (end 142.875 81.661) (width 0.3) (layer F.Cu) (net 3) (status 10))
 (segment (start 153.162 85.979) (end 153.162 86.487) (width 0.3) (layer F.Cu) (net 3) (status 30))
 (segment (start 150.862 83.679) (end 153.162 85.979) (width 0.3) (layer F.Cu) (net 3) (status 20))
 (segment (start 142.875 83.820002) (end 143.763999 84.709001) (width 0.3) (layer B.Cu) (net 3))
 (segment (start 142.875 81.661) (end 142.875 83.820002) (width 0.3) (layer B.Cu) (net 3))
 (via (at 143.763999 84.709001) (size 0.7) (drill 0.4) (layers F.Cu B.Cu) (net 3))
 (segment (start 144.893974 84.074) (end 144.258973 84.709001) (width 0.3) (layer F.Cu) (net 3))
 (segment (start 144.258973 84.709001) (end 143.763999 84.709001) (width 0.3) (layer F.Cu) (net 3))
 (segment (start 149.465 84.074) (end 144.893974 84.074) (width 0.3) (layer F.Cu) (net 3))
 (segment (start 150.467 83.679) (end 149.606705 82.818705) (width 0.3) (layer F.Cu) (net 3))
 (segment (start 150.862 83.679) (end 150.467 83.679) (width 0.3) (layer F.Cu) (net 3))
 (segment (start 149.465 82.96041) (end 149.606705 82.818705) (width 0.3) (layer F.Cu) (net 3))
 (segment (start 149.465 84.074) (end 149.465 82.96041) (width 0.3) (layer F.Cu) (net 3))
 (segment (start 143.724 94.869) (end 145.019001 96.164001) (width 0.25) (layer F.Cu) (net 9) (status 20))
 (segment (start 140.710998 94.869) (end 143.724 94.869) (width 0.25) (layer F.Cu) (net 9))
 (segment (start 139.192 92.87) (end 139.192 93.350002) (width 0.25) (layer F.Cu) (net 9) (status 30))
 (segment (start 139.192 93.350002) (end 140.710998 94.869) (width 0.25) (layer F.Cu) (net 9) (status 10))
 (segment (start 145.216 94.361) (end 147.019001 96.164001) (width 0.25) (layer F.Cu) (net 8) (status 20))
 (segment (start 141.478 94.361) (end 145.216 94.361) (width 0.25) (layer F.Cu) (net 8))
 (segment (start 140.462 92.87) (end 140.462 93.345) (width 0.25) (layer F.Cu) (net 8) (status 30))
 (segment (start 140.462 93.345) (end 141.478 94.361) (width 0.25) (layer F.Cu) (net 8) (status 10))
 (segment (start 146.558 92.964) (end 148.491 92.964) (width 0.2) (layer F.Cu) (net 10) (status 30))
 (segment (start 140.194 82.677) (end 142 82.677) (width 0.2) (layer F.Cu) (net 12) (status 30))
 (segment (start 147.715 82.677) (end 148.858 81.534) (width 0.2) (layer F.Cu) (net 11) (status 1000000))
 (segment (start 152.333 80.885) (end 152.908 80.885) (width 0.2) (layer F.Cu) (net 11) (status 1000000))
 (segment (start 148.858 81.534) (end 151.684 81.534) (width 0.2) (layer F.Cu) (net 11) (status 1000000))
 (segment (start 151.684 81.534) (end 152.333 80.885) (width 0.2) (layer F.Cu) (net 11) (status 1000000))
 (segment (start 151.948002 93.735) (end 152.654 93.735) (width 0.3) (layer F.Cu) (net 7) (status 20))
 (segment (start 149.519001 96.164001) (end 151.948002 93.735) (width 0.3) (layer F.Cu) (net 7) (status 10))
 (segment (start 140.462 84.977) (end 140.194 84.709) (width 0.2) (layer F.Cu) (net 5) (status 30))
 (segment (start 140.462 87.47) (end 140.462 84.977) (width 0.2) (layer F.Cu) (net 5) (status 30))
 (segment (start 141.718 84.709) (end 143.75 82.677) (width 0.2) (layer F.Cu) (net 5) (status 20))
 (segment (start 140.194 84.709) (end 141.718 84.709) (width 0.2) (layer F.Cu) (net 5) (status 10))
 (segment (start 143.75 80.405) (end 144.272 79.883) (width 0.2) (layer F.Cu) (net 5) (status 30))
 (segment (start 143.75 82.677) (end 143.75 80.405) (width 0.2) (layer F.Cu) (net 5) (status 30))
 (segment (start 145.962001 80.732999) (end 146.812 79.883) (width 0.2) (layer F.Cu) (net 6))
 (segment (start 145.056928 81.638072) (end 145.962001 80.732999) (width 0.2) (layer F.Cu) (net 6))
 (segment (start 145.556 82.677) (end 145.056928 82.177928) (width 0.2) (layer F.Cu) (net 6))
 (segment (start 145.056928 83.176072) (end 145.556 82.677) (width 0.2) (layer F.Cu) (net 6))
 (segment (start 144.915928 83.176072) (end 145.056928 83.176072) (width 0.2) (layer F.Cu) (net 6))
 (segment (start 144.287001 83.804999) (end 144.915928 83.176072) (width 0.2) (layer F.Cu) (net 6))
 (segment (start 143.705999 83.804999) (end 144.287001 83.804999) (width 0.2) (layer F.Cu) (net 6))
 (segment (start 141.732 85.778998) (end 143.705999 83.804999) (width 0.2) (layer F.Cu) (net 6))
 (segment (start 145.056928 82.177928) (end 145.056928 81.638072) (width 0.2) (layer F.Cu) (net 6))
 (segment (start 141.732 87.47) (end 141.732 85.778998) (width 0.2) (layer F.Cu) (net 6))
 (segment (start 148.209 78.486) (end 152.259 78.486) (width 0.2) (layer F.Cu) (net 6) (status 1000000))
 (segment (start 152.259 78.486) (end 152.908 79.135) (width 0.2) (layer F.Cu) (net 6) (status 1000000))
 (segment (start 146.812 79.883) (end 148.209 78.486) (width 0.2) (layer F.Cu) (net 6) (status 1000000))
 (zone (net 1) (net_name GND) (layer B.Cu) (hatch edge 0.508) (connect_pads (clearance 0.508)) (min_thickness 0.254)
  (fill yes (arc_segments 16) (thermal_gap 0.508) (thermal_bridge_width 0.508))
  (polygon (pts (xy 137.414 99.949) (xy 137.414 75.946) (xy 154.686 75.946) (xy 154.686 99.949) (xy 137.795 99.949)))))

